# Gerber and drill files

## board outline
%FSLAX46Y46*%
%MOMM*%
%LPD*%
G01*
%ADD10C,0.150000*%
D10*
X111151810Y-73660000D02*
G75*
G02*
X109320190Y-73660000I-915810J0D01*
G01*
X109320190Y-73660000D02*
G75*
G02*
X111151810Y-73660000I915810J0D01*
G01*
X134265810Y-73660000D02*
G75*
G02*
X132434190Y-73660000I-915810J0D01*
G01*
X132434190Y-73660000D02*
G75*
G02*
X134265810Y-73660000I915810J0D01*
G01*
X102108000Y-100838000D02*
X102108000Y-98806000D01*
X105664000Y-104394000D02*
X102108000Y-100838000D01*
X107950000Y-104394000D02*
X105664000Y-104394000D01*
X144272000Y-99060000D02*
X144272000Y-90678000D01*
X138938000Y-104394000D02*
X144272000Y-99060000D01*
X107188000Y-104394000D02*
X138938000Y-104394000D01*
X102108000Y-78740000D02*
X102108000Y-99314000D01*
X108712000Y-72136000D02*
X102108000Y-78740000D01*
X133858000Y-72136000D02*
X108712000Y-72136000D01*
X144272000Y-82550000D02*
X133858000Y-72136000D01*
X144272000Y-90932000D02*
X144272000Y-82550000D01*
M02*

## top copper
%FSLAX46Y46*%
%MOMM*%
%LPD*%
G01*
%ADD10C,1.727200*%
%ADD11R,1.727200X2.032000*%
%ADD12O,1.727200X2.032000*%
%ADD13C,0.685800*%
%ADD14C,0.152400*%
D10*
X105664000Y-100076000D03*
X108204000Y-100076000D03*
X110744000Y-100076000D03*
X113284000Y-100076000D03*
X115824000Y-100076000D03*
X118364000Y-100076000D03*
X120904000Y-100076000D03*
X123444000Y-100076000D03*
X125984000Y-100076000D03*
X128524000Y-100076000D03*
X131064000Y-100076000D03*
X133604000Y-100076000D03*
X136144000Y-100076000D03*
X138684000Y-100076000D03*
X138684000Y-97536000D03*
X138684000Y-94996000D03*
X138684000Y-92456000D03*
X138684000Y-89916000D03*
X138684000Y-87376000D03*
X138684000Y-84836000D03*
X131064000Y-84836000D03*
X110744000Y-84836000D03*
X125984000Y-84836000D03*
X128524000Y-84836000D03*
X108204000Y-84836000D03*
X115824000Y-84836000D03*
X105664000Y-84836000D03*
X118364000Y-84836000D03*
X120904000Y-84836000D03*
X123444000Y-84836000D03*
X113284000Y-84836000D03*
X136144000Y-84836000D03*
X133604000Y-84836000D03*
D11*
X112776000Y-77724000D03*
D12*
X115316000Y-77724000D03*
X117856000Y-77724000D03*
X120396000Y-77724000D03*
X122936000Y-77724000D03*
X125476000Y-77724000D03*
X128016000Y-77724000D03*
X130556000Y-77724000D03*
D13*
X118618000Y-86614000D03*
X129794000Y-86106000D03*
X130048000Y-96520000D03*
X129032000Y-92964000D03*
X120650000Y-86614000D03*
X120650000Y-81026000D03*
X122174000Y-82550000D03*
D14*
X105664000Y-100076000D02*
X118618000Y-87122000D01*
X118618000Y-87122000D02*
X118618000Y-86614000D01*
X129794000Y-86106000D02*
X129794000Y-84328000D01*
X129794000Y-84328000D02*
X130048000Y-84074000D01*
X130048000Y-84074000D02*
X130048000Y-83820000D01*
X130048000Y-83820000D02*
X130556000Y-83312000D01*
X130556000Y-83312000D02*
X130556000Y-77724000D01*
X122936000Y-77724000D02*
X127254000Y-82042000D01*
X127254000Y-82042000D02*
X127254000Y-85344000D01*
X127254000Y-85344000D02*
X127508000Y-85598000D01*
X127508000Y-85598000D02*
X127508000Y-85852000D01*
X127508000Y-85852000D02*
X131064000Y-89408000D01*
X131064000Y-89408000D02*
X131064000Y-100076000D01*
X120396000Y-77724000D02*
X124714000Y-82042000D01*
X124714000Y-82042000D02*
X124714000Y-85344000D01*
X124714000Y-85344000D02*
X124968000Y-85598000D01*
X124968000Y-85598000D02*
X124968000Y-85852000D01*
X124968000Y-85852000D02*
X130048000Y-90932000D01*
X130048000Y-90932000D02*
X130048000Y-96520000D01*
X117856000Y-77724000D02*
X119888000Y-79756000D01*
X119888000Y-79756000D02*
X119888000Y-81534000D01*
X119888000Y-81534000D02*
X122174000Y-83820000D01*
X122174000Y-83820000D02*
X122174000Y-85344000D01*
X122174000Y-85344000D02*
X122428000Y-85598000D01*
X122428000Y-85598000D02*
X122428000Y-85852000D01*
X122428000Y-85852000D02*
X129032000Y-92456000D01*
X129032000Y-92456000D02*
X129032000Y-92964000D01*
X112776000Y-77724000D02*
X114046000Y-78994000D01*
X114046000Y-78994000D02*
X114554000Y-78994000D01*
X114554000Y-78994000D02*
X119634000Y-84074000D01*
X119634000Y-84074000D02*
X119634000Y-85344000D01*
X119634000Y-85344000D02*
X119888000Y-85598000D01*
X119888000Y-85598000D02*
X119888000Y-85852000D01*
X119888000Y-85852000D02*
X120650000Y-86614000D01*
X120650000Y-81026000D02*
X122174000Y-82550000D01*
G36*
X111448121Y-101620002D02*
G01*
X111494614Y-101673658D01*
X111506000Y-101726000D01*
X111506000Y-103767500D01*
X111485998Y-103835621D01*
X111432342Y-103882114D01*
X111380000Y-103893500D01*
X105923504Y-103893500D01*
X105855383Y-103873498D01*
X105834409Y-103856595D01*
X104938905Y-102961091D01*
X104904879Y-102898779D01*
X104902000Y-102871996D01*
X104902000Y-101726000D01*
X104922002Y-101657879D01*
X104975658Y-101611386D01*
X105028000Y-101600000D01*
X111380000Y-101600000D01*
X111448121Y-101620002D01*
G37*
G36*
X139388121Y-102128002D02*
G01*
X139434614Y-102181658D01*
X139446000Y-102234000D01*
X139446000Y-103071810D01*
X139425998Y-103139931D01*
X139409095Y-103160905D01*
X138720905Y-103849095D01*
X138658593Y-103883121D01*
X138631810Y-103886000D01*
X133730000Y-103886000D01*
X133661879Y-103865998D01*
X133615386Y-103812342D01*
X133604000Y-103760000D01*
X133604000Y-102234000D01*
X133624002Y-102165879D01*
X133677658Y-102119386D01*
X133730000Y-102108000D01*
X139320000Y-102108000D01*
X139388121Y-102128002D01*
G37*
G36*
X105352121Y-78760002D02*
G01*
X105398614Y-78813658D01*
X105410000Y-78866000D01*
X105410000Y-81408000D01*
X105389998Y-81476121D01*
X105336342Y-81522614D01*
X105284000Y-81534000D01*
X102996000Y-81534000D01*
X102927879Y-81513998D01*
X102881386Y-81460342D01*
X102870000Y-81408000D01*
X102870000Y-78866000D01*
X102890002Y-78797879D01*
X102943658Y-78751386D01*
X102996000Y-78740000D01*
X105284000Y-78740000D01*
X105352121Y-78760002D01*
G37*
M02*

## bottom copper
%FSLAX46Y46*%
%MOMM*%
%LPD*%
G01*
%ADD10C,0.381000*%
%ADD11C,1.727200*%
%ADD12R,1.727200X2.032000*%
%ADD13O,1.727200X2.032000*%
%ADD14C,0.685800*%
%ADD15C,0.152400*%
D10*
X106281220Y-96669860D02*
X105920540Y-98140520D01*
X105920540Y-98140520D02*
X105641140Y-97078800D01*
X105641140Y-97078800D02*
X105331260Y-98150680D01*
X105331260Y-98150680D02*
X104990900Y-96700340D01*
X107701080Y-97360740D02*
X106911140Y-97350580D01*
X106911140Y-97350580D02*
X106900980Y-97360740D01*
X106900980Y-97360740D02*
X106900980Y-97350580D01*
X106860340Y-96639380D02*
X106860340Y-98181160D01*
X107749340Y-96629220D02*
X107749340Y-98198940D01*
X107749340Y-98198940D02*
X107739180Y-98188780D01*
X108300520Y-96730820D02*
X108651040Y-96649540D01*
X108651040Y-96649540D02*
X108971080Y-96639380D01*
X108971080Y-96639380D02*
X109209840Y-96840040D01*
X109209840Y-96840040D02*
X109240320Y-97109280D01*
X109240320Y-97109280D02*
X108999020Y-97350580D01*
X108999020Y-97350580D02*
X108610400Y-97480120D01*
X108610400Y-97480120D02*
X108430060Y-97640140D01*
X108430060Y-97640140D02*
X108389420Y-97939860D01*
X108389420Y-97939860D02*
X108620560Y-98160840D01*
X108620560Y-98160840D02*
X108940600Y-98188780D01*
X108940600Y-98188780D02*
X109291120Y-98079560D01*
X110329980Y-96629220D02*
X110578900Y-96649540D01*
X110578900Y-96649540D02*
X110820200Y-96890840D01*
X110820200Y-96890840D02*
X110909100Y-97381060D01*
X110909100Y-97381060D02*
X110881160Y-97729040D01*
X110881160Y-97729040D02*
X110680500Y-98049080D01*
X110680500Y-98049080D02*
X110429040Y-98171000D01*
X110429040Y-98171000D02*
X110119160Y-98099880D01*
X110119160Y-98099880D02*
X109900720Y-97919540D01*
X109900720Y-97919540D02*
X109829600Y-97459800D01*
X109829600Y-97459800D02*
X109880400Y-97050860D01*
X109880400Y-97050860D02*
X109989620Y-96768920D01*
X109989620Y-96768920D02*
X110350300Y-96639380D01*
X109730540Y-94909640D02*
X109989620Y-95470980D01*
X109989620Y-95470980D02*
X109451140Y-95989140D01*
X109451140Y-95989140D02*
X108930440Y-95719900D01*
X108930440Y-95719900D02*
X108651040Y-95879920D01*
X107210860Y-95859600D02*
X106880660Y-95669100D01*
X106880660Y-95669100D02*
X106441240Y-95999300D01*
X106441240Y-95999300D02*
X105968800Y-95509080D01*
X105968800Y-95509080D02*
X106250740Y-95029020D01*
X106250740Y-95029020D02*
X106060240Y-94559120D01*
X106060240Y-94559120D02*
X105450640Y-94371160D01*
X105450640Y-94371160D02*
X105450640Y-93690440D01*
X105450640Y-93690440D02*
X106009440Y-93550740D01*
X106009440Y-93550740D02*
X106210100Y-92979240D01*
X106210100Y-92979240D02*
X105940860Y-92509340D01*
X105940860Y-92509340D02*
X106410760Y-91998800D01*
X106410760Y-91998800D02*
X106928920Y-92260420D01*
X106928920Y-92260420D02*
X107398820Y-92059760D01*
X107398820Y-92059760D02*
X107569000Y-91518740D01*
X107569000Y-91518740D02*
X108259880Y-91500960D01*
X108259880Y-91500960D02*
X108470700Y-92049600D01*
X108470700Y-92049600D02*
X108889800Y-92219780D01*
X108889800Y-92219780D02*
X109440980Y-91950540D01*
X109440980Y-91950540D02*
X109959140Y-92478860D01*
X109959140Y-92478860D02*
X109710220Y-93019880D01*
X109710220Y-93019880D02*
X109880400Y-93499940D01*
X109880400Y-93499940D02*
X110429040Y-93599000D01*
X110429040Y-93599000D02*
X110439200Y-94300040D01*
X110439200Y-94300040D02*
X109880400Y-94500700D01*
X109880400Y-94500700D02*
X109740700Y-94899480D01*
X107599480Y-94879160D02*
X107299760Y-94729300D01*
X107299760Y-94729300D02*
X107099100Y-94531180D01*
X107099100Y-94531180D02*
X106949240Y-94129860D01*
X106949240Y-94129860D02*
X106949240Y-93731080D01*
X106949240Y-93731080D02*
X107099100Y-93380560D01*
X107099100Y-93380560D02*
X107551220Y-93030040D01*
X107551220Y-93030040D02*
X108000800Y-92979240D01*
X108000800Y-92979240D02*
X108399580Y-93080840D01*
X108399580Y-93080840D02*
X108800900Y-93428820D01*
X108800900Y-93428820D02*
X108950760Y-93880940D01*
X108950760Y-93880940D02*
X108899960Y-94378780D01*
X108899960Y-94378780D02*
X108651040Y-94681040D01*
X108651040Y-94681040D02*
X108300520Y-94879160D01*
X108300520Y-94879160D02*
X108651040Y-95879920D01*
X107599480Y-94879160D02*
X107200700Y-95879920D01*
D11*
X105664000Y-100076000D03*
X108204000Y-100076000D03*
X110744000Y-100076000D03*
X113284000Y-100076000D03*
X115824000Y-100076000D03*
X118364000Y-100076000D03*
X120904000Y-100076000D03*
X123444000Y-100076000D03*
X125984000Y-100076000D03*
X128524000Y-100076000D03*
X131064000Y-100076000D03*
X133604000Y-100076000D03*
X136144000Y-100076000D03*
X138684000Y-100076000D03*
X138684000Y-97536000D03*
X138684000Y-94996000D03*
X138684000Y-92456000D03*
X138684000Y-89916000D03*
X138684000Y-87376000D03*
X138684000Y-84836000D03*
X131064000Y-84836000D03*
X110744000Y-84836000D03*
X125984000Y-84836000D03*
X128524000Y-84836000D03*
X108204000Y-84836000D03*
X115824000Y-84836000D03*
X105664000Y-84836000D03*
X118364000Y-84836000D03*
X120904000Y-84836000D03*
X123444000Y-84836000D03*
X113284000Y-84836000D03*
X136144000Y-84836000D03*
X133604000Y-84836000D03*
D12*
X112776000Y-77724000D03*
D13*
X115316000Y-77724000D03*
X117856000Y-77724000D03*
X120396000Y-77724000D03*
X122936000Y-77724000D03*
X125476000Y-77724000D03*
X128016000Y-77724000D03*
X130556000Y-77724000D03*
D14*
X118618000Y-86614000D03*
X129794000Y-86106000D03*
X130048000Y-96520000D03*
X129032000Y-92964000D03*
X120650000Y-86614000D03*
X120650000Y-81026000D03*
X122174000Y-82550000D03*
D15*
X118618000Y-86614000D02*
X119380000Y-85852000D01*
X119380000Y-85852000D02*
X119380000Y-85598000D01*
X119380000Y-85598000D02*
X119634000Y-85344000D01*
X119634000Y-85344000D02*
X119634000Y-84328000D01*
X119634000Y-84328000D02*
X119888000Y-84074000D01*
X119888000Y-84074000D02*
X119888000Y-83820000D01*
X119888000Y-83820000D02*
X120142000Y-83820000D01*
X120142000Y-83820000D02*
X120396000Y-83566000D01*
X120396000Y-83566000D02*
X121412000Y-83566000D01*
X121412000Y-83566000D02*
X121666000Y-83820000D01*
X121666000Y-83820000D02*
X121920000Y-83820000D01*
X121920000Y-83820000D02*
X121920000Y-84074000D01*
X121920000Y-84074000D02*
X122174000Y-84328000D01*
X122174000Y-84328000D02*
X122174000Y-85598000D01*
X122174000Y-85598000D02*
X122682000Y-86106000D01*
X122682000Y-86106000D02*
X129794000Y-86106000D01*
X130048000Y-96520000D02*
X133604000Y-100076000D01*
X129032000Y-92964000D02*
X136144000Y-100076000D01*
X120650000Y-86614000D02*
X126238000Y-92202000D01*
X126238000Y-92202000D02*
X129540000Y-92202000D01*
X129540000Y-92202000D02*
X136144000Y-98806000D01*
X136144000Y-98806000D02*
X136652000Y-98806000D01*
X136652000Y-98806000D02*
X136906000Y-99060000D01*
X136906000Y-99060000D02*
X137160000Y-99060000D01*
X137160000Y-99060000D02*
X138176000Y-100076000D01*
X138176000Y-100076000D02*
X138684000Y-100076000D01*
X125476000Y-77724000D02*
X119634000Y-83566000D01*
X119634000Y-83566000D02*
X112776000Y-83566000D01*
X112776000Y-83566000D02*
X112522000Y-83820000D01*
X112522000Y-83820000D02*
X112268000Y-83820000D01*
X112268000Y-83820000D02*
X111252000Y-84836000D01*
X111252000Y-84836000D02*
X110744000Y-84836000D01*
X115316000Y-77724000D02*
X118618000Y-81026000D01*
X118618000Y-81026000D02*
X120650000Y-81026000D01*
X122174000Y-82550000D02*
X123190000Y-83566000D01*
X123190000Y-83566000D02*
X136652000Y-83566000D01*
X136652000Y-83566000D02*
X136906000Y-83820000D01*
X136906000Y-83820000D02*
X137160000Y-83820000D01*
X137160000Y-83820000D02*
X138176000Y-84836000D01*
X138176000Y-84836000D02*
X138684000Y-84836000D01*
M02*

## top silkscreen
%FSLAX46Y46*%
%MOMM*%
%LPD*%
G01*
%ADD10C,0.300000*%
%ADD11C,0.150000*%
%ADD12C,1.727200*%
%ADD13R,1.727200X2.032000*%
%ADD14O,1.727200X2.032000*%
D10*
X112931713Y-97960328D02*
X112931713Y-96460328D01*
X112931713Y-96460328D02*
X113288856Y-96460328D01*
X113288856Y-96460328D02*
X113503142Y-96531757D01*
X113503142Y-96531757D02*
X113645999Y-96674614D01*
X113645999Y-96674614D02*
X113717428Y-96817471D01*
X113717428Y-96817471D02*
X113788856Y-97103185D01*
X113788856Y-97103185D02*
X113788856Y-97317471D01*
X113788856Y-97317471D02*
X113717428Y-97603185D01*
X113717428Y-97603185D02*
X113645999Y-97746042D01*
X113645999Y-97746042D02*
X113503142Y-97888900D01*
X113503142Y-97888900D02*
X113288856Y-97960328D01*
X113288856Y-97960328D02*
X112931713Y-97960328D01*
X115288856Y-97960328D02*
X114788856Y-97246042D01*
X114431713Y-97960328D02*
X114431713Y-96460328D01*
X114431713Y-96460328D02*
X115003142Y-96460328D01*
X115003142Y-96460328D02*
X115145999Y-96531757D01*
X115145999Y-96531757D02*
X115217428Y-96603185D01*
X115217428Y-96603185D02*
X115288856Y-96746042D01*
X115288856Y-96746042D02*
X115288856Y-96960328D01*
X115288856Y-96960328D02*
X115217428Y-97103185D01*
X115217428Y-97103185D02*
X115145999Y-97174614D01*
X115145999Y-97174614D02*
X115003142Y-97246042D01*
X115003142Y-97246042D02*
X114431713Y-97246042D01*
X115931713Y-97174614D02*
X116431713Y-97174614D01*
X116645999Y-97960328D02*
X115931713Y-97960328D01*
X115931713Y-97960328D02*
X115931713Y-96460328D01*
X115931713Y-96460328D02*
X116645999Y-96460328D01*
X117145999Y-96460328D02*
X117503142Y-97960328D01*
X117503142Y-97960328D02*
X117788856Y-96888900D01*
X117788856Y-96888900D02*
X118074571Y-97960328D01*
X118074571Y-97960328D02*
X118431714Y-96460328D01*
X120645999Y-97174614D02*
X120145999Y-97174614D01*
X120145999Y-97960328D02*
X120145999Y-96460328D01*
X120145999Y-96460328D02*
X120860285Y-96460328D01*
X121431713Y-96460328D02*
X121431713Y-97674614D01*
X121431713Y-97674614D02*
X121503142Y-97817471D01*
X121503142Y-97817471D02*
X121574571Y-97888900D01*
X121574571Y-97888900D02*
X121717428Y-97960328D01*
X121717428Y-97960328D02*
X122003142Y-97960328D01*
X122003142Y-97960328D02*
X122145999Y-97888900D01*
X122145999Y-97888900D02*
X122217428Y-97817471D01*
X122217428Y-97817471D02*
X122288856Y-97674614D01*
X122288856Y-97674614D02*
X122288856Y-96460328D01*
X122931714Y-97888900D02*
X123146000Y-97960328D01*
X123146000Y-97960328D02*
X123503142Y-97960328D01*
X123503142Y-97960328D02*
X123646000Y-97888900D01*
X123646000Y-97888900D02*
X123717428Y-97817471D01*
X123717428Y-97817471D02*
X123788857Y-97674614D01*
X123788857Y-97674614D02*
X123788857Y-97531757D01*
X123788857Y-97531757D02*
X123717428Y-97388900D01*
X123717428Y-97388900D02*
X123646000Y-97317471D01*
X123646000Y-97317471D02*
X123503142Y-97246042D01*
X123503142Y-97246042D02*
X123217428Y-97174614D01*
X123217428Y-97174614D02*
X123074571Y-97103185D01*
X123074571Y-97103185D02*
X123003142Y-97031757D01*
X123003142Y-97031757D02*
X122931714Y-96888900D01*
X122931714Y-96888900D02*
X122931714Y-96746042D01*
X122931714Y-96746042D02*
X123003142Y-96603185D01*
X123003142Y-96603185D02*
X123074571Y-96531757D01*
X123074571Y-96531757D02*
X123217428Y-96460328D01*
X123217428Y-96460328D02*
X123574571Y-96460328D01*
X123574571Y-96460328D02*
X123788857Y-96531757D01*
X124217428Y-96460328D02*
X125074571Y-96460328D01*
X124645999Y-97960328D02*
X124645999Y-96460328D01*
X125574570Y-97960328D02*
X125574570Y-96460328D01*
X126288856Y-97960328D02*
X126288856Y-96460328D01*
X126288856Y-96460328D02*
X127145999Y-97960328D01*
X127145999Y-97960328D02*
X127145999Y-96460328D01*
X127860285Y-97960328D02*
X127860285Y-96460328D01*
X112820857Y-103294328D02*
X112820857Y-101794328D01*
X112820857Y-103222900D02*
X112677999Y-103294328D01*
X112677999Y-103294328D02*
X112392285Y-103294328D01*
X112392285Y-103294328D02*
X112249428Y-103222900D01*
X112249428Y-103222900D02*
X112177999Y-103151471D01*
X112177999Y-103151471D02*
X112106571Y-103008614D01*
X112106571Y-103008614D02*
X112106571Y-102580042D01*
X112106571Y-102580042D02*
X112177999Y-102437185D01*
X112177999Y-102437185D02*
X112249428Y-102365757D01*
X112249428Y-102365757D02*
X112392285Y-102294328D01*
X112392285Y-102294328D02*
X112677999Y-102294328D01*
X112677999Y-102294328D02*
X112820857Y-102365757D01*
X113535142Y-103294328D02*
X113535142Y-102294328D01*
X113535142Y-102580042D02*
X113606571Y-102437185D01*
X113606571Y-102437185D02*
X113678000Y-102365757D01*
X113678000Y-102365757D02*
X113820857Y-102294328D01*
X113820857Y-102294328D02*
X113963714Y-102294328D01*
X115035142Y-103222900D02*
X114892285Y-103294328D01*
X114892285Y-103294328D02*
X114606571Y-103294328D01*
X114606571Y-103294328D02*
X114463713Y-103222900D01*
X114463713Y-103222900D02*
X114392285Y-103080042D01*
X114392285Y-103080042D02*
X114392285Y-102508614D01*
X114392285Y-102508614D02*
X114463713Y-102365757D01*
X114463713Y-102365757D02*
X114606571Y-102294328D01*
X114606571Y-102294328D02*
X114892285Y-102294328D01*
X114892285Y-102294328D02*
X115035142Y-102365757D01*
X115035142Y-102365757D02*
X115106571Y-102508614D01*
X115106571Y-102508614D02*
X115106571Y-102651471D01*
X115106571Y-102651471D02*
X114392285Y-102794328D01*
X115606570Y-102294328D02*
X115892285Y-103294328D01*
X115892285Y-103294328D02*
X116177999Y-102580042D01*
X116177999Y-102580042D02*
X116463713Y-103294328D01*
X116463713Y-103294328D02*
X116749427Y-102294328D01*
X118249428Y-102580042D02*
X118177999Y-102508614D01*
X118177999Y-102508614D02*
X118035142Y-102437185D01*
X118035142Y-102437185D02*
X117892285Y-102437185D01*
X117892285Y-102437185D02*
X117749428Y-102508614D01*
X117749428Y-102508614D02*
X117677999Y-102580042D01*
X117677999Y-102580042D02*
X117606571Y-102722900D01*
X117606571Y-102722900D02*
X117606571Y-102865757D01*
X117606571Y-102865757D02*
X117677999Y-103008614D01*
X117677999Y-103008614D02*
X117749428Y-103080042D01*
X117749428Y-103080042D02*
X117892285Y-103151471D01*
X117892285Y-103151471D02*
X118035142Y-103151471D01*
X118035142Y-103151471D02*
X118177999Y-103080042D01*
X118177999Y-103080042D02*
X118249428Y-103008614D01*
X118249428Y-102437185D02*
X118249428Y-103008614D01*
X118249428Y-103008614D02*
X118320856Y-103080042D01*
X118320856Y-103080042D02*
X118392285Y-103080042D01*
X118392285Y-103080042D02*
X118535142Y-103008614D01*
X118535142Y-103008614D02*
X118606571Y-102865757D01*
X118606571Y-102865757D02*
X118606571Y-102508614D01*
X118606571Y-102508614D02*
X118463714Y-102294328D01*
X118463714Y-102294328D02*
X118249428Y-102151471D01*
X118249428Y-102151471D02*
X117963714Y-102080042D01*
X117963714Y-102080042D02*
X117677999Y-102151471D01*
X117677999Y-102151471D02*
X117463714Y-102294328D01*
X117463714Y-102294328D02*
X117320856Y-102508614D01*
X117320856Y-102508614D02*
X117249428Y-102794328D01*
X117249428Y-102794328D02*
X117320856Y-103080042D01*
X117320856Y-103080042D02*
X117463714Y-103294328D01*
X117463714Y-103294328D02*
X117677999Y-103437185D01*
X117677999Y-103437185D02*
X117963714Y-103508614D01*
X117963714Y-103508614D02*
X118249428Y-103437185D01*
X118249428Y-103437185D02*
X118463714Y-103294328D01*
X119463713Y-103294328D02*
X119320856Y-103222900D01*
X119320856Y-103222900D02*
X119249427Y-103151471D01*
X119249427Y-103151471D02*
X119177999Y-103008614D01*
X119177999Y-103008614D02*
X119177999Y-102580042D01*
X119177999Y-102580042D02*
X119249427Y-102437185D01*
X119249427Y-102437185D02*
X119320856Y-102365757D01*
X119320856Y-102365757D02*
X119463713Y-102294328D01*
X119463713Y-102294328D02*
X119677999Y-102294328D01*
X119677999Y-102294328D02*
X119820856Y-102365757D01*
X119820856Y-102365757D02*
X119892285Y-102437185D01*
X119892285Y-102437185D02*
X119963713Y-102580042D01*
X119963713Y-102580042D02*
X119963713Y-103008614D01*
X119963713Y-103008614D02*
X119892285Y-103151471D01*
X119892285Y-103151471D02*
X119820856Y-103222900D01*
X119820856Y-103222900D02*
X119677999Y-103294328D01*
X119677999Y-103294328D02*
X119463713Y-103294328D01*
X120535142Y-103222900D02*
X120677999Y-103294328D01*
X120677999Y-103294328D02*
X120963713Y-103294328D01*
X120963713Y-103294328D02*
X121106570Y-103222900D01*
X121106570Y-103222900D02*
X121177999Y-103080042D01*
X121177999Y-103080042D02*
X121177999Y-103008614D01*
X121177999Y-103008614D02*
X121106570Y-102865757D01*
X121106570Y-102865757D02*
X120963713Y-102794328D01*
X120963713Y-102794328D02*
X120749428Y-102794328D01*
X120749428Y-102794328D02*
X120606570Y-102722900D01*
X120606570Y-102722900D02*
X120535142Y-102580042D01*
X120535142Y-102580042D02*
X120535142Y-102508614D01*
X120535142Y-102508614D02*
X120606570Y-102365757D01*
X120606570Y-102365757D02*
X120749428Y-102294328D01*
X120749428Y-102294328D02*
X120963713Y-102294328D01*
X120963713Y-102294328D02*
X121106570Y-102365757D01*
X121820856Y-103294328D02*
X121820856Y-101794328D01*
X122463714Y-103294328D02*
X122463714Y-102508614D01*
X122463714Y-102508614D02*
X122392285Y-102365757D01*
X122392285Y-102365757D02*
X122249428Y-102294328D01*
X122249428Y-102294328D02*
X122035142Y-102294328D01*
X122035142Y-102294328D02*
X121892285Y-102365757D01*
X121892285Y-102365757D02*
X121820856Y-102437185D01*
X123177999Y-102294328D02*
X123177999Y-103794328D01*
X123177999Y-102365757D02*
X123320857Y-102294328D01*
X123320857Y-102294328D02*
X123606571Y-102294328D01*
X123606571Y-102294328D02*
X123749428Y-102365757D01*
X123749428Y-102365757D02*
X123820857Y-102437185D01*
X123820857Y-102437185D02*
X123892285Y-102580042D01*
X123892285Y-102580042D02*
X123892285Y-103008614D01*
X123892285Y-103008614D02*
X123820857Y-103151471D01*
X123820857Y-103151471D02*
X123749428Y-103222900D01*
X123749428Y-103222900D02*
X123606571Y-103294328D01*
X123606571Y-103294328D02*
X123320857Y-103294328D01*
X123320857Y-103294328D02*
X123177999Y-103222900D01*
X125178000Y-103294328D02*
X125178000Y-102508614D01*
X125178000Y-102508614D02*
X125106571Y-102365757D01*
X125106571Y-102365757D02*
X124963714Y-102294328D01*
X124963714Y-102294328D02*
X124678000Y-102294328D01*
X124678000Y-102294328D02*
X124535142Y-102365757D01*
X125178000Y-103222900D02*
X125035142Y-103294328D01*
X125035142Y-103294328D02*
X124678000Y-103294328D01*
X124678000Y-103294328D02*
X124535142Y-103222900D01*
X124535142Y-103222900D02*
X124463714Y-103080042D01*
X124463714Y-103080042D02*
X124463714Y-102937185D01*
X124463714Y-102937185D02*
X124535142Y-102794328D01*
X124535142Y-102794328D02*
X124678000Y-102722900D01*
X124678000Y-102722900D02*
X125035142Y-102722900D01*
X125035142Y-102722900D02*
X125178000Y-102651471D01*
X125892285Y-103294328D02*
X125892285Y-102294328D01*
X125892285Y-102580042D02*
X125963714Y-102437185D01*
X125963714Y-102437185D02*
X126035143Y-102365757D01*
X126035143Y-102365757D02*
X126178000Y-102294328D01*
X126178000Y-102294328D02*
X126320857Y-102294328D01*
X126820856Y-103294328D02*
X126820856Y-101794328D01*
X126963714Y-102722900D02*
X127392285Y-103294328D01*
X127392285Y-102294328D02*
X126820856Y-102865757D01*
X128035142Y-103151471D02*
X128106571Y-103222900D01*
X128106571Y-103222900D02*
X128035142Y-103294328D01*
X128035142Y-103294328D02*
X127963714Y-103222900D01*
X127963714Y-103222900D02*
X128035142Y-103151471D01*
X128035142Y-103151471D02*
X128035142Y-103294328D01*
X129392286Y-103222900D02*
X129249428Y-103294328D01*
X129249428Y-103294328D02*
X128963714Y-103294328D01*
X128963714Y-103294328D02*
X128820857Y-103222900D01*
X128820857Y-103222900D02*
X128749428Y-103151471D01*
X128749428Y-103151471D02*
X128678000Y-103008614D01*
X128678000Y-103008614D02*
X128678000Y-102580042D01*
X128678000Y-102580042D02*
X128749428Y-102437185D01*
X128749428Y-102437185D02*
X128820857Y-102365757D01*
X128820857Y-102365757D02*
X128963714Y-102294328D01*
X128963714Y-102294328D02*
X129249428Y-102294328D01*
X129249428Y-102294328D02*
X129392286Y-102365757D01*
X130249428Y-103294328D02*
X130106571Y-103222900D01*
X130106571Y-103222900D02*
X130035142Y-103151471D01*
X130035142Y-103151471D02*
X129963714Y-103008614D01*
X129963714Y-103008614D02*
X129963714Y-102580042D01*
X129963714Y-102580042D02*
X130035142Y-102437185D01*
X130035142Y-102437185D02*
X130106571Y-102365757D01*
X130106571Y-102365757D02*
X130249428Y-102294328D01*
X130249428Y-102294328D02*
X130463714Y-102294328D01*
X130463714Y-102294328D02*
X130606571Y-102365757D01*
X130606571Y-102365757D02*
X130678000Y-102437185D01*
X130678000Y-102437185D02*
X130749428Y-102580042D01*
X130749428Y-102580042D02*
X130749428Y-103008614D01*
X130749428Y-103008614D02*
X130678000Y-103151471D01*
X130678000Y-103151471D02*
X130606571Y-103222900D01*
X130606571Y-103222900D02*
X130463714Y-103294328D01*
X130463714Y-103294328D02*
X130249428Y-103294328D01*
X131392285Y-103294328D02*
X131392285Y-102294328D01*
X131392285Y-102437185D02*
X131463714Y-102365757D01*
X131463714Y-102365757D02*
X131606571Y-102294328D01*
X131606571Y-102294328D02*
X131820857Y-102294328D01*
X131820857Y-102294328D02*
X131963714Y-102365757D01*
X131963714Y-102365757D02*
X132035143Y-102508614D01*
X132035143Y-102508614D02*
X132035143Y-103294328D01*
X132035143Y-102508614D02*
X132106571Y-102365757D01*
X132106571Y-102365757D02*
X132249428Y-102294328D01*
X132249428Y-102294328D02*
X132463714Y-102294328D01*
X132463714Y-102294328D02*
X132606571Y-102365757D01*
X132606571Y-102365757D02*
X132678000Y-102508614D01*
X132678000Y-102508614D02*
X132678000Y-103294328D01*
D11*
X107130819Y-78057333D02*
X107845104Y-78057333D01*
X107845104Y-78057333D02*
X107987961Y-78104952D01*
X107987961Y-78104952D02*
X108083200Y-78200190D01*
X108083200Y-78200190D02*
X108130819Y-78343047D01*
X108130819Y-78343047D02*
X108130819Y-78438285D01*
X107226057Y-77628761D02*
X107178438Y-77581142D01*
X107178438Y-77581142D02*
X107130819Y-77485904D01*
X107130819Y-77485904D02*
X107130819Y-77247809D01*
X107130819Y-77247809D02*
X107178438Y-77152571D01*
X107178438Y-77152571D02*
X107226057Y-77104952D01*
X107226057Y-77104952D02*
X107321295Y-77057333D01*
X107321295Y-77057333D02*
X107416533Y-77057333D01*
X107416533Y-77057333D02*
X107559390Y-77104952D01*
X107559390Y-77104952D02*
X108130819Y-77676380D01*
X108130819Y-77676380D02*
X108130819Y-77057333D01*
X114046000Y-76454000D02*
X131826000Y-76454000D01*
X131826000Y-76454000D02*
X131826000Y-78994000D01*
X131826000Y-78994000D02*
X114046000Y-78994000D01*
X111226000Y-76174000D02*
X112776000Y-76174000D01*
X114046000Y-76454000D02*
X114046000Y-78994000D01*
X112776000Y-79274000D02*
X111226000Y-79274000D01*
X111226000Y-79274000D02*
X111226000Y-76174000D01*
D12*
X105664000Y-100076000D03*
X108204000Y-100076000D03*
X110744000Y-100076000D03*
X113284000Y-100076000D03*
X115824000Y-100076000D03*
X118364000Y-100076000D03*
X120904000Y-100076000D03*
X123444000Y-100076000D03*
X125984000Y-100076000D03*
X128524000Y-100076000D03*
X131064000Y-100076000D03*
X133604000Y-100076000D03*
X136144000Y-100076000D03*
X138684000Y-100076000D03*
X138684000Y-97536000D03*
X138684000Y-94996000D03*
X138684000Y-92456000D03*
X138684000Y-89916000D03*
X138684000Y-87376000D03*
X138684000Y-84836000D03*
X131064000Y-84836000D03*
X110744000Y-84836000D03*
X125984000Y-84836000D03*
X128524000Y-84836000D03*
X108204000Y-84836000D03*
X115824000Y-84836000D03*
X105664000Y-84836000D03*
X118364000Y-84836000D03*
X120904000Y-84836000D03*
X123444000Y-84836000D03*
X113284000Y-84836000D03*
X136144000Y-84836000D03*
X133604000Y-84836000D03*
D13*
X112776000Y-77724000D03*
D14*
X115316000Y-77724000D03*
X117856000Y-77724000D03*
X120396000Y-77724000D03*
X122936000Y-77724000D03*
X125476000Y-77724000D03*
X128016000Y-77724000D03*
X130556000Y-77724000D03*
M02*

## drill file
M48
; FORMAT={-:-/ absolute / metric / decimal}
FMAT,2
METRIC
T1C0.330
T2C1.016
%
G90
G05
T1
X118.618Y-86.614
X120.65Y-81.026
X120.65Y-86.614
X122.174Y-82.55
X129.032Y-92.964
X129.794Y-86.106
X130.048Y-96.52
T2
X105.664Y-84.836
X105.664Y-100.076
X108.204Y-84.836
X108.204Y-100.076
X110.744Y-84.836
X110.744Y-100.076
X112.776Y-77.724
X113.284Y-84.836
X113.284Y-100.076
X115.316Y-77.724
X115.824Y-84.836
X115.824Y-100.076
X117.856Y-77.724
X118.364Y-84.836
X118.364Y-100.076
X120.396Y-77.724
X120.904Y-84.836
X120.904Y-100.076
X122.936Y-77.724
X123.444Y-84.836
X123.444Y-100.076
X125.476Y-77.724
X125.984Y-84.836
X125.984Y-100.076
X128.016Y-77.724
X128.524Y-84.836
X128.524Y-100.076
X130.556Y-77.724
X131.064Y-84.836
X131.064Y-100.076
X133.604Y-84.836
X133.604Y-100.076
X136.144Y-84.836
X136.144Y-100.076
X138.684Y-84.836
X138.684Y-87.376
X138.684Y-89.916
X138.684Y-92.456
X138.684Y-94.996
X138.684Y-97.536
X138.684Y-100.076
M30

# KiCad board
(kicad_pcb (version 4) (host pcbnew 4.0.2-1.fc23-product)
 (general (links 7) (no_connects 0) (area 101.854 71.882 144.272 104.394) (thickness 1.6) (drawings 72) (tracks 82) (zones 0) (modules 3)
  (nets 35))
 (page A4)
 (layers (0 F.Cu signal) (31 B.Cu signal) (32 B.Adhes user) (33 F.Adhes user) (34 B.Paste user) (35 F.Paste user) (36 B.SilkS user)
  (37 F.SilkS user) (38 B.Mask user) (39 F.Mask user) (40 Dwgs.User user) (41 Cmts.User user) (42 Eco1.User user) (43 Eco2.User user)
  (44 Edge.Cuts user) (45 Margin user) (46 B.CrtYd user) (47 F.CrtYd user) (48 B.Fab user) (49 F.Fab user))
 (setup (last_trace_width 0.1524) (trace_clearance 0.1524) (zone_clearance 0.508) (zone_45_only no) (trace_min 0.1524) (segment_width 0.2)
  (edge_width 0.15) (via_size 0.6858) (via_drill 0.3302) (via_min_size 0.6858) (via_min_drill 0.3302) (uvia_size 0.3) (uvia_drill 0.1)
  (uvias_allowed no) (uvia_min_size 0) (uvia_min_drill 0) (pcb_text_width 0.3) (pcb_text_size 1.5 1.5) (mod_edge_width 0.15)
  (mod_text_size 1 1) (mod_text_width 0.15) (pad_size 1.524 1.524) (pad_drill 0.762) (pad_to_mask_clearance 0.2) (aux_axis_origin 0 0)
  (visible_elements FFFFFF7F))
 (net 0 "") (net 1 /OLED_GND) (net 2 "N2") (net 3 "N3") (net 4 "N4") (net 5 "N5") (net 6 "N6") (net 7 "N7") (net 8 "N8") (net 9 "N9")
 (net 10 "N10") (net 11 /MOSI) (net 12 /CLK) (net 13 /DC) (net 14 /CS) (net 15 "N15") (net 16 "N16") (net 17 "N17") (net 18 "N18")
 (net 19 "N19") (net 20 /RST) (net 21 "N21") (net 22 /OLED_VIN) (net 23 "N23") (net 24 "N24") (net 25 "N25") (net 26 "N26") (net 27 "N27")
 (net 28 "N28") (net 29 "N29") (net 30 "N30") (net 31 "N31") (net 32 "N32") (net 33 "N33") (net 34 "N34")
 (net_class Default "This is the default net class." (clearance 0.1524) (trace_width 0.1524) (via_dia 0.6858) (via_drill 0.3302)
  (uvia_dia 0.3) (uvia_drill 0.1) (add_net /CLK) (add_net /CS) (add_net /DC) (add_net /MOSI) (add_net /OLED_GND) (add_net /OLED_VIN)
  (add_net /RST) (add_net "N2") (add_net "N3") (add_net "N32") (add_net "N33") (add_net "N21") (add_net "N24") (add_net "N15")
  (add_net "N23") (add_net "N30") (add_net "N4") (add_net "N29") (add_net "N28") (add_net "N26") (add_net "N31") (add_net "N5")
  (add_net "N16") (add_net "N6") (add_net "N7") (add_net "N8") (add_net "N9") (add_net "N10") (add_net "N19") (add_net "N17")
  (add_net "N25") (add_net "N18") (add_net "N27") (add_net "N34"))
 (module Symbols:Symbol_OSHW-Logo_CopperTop (layer B.Cu) (at 107.95 93.98 180)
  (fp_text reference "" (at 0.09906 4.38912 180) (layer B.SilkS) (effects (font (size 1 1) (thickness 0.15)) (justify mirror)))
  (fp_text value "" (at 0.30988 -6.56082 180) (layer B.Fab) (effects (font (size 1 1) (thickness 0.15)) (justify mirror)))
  (fp_line (start 1.66878 -2.68986) (end 2.02946 -4.16052) (layer B.Cu) (width 0.381))
  (fp_line (start 2.02946 -4.16052) (end 2.30886 -3.0988) (layer B.Cu) (width 0.381))
  (fp_line (start 2.30886 -3.0988) (end 2.61874 -4.17068) (layer B.Cu) (width 0.381))
  (fp_line (start 2.61874 -4.17068) (end 2.9591 -2.72034) (layer B.Cu) (width 0.381))
  (fp_line (start 0.24892 -3.38074) (end 1.03886 -3.37058) (layer B.Cu) (width 0.381))
  (fp_line (start 1.03886 -3.37058) (end 1.04902 -3.38074) (layer B.Cu) (width 0.381))
  (fp_line (start 1.04902 -3.38074) (end 1.04902 -3.37058) (layer B.Cu) (width 0.381))
  (fp_line (start 1.08966 -2.65938) (end 1.08966 -4.20116) (layer B.Cu) (width 0.381))
  (fp_line (start 0.20066 -2.64922) (end 0.20066 -4.21894) (layer B.Cu) (width 0.381))
  (fp_line (start 0.20066 -4.21894) (end 0.21082 -4.20878) (layer B.Cu) (width 0.381))
  (fp_line (start -0.35052 -2.75082) (end -0.70104 -2.66954) (layer B.Cu) (width 0.381))
  (fp_line (start -0.70104 -2.66954) (end -1.02108 -2.65938) (layer B.Cu) (width 0.381))
  (fp_line (start -1.02108 -2.65938) (end -1.25984 -2.86004) (layer B.Cu) (width 0.381))
  (fp_line (start -1.25984 -2.86004) (end -1.29032 -3.12928) (layer B.Cu) (width 0.381))
  (fp_line (start -1.29032 -3.12928) (end -1.04902 -3.37058) (layer B.Cu) (width 0.381))
  (fp_line (start -1.04902 -3.37058) (end -0.6604 -3.50012) (layer B.Cu) (width 0.381))
  (fp_line (start -0.6604 -3.50012) (end -0.48006 -3.66014) (layer B.Cu) (width 0.381))
  (fp_line (start -0.48006 -3.66014) (end -0.43942 -3.95986) (layer B.Cu) (width 0.381))
  (fp_line (start -0.43942 -3.95986) (end -0.67056 -4.18084) (layer B.Cu) (width 0.381))
  (fp_line (start -0.67056 -4.18084) (end -0.9906 -4.20878) (layer B.Cu) (width 0.381))
  (fp_line (start -0.9906 -4.20878) (end -1.34112 -4.09956) (layer B.Cu) (width 0.381))
  (fp_line (start -2.37998 -2.64922) (end -2.6289 -2.66954) (layer B.Cu) (width 0.381))
  (fp_line (start -2.6289 -2.66954) (end -2.8702 -2.91084) (layer B.Cu) (width 0.381))
  (fp_line (start -2.8702 -2.91084) (end -2.9591 -3.40106) (layer B.Cu) (width 0.381))
  (fp_line (start -2.9591 -3.40106) (end -2.93116 -3.74904) (layer B.Cu) (width 0.381))
  (fp_line (start -2.93116 -3.74904) (end -2.7305 -4.06908) (layer B.Cu) (width 0.381))
  (fp_line (start -2.7305 -4.06908) (end -2.47904 -4.191) (layer B.Cu) (width 0.381))
  (fp_line (start -2.47904 -4.191) (end -2.16916 -4.11988) (layer B.Cu) (width 0.381))
  (fp_line (start -2.16916 -4.11988) (end -1.95072 -3.93954) (layer B.Cu) (width 0.381))
  (fp_line (start -1.95072 -3.93954) (end -1.8796 -3.4798) (layer B.Cu) (width 0.381))
  (fp_line (start -1.8796 -3.4798) (end -1.9304 -3.07086) (layer B.Cu) (width 0.381))
  (fp_line (start -1.9304 -3.07086) (end -2.03962 -2.78892) (layer B.Cu) (width 0.381))
  (fp_line (start -2.03962 -2.78892) (end -2.4003 -2.65938) (layer B.Cu) (width 0.381))
  (fp_line (start -1.78054 -0.92964) (end -2.03962 -1.49098) (layer B.Cu) (width 0.381))
  (fp_line (start -2.03962 -1.49098) (end -1.50114 -2.00914) (layer B.Cu) (width 0.381))
  (fp_line (start -1.50114 -2.00914) (end -0.98044 -1.7399) (layer B.Cu) (width 0.381))
  (fp_line (start -0.98044 -1.7399) (end -0.70104 -1.89992) (layer B.Cu) (width 0.381))
  (fp_line (start 0.73914 -1.8796) (end 1.06934 -1.6891) (layer B.Cu) (width 0.381))
  (fp_line (start 1.06934 -1.6891) (end 1.50876 -2.0193) (layer B.Cu) (width 0.381))
  (fp_line (start 1.50876 -2.0193) (end 1.9812 -1.52908) (layer B.Cu) (width 0.381))
  (fp_line (start 1.9812 -1.52908) (end 1.69926 -1.04902) (layer B.Cu) (width 0.381))
  (fp_line (start 1.69926 -1.04902) (end 1.88976 -0.57912) (layer B.Cu) (width 0.381))
  (fp_line (start 1.88976 -0.57912) (end 2.49936 -0.39116) (layer B.Cu) (width 0.381))
  (fp_line (start 2.49936 -0.39116) (end 2.49936 0.28956) (layer B.Cu) (width 0.381))
  (fp_line (start 2.49936 0.28956) (end 1.94056 0.42926) (layer B.Cu) (width 0.381))
  (fp_line (start 1.94056 0.42926) (end 1.7399 1.00076) (layer B.Cu) (width 0.381))
  (fp_line (start 1.7399 1.00076) (end 2.00914 1.47066) (layer B.Cu) (width 0.381))
  (fp_line (start 2.00914 1.47066) (end 1.53924 1.9812) (layer B.Cu) (width 0.381))
  (fp_line (start 1.53924 1.9812) (end 1.02108 1.71958) (layer B.Cu) (width 0.381))
  (fp_line (start 1.02108 1.71958) (end 0.55118 1.92024) (layer B.Cu) (width 0.381))
  (fp_line (start 0.55118 1.92024) (end 0.381 2.46126) (layer B.Cu) (width 0.381))
  (fp_line (start 0.381 2.46126) (end -0.30988 2.47904) (layer B.Cu) (width 0.381))
  (fp_line (start -0.30988 2.47904) (end -0.5207 1.9304) (layer B.Cu) (width 0.381))
  (fp_line (start -0.5207 1.9304) (end -0.9398 1.76022) (layer B.Cu) (width 0.381))
  (fp_line (start -0.9398 1.76022) (end -1.49098 2.02946) (layer B.Cu) (width 0.381))
  (fp_line (start -1.49098 2.02946) (end -2.00914 1.50114) (layer B.Cu) (width 0.381))
  (fp_line (start -2.00914 1.50114) (end -1.76022 0.96012) (layer B.Cu) (width 0.381))
  (fp_line (start -1.76022 0.96012) (end -1.9304 0.48006) (layer B.Cu) (width 0.381))
  (fp_line (start -1.9304 0.48006) (end -2.47904 0.381) (layer B.Cu) (width 0.381))
  (fp_line (start -2.47904 0.381) (end -2.4892 -0.32004) (layer B.Cu) (width 0.381))
  (fp_line (start -2.4892 -0.32004) (end -1.9304 -0.5207) (layer B.Cu) (width 0.381))
  (fp_line (start -1.9304 -0.5207) (end -1.7907 -0.91948) (layer B.Cu) (width 0.381))
  (fp_line (start 0.35052 -0.89916) (end 0.65024 -0.7493) (layer B.Cu) (width 0.381))
  (fp_line (start 0.65024 -0.7493) (end 0.8509 -0.55118) (layer B.Cu) (width 0.381))
  (fp_line (start 0.8509 -0.55118) (end 1.00076 -0.14986) (layer B.Cu) (width 0.381))
  (fp_line (start 1.00076 -0.14986) (end 1.00076 0.24892) (layer B.Cu) (width 0.381))
  (fp_line (start 1.00076 0.24892) (end 0.8509 0.59944) (layer B.Cu) (width 0.381))
  (fp_line (start 0.8509 0.59944) (end 0.39878 0.94996) (layer B.Cu) (width 0.381))
  (fp_line (start 0.39878 0.94996) (end -0.0508 1.00076) (layer B.Cu) (width 0.381))
  (fp_line (start -0.0508 1.00076) (end -0.44958 0.89916) (layer B.Cu) (width 0.381))
  (fp_line (start -0.44958 0.89916) (end -0.8509 0.55118) (layer B.Cu) (width 0.381))
  (fp_line (start -0.8509 0.55118) (end -1.00076 0.09906) (layer B.Cu) (width 0.381))
  (fp_line (start -1.00076 0.09906) (end -0.94996 -0.39878) (layer B.Cu) (width 0.381))
  (fp_line (start -0.94996 -0.39878) (end -0.70104 -0.70104) (layer B.Cu) (width 0.381))
  (fp_line (start -0.70104 -0.70104) (end -0.35052 -0.89916) (layer B.Cu) (width 0.381))
  (fp_line (start -0.35052 -0.89916) (end -0.70104 -1.89992) (layer B.Cu) (width 0.381))
  (fp_line (start 0.35052 -0.89916) (end 0.7493 -1.89992) (layer B.Cu) (width 0.381)))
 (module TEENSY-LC (layer F.Cu) (at 115.824 89.916 90)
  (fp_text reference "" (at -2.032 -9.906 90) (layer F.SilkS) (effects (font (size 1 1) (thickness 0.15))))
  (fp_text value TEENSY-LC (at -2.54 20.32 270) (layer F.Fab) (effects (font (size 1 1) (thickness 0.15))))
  (pad G1 thru_hole circle (at -10.16 -10.16 90) (size 1.7272 1.7272) (drill 1.016) (layers *.Cu *.Mask F.SilkS) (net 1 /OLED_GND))
  (pad 0 thru_hole circle (at -10.16 -7.62 90) (size 1.7272 1.7272) (drill 1.016) (layers *.Cu *.Mask F.SilkS) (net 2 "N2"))
  (pad 1 thru_hole circle (at -10.16 -5.08 90) (size 1.7272 1.7272) (drill 1.016) (layers *.Cu *.Mask F.SilkS) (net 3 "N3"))
  (pad 2 thru_hole circle (at -10.16 -2.54 90) (size 1.7272 1.7272) (drill 1.016) (layers *.Cu *.Mask F.SilkS) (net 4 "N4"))
  (pad 3 thru_hole circle (at -10.16 0 90) (size 1.7272 1.7272) (drill 1.016) (layers *.Cu *.Mask F.SilkS) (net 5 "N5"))
  (pad 4 thru_hole circle (at -10.16 2.54 90) (size 1.7272 1.7272) (drill 1.016) (layers *.Cu *.Mask F.SilkS) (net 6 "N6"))
  (pad 5 thru_hole circle (at -10.16 5.08 90) (size 1.7272 1.7272) (drill 1.016) (layers *.Cu *.Mask F.SilkS) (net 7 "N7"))
  (pad 6 thru_hole circle (at -10.16 7.62 90) (size 1.7272 1.7272) (drill 1.016) (layers *.Cu *.Mask F.SilkS) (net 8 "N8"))
  (pad 7 thru_hole circle (at -10.16 10.16 90) (size 1.7272 1.7272) (drill 1.016) (layers *.Cu *.Mask F.SilkS) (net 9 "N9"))
  (pad 8 thru_hole circle (at -10.16 12.7 90) (size 1.7272 1.7272) (drill 1.016) (layers *.Cu *.Mask F.SilkS) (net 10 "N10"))
  (pad 9 thru_hole circle (at -10.16 15.24 90) (size 1.7272 1.7272) (drill 1.016) (layers *.Cu *.Mask F.SilkS) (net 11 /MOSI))
  (pad 10 thru_hole circle (at -10.16 17.78 90) (size 1.7272 1.7272) (drill 1.016) (layers *.Cu *.Mask F.SilkS) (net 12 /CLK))
  (pad 11 thru_hole circle (at -10.16 20.32 90) (size 1.7272 1.7272) (drill 1.016) (layers *.Cu *.Mask F.SilkS) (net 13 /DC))
  (pad 12 thru_hole circle (at -10.16 22.86 90) (size 1.7272 1.7272) (drill 1.016) (layers *.Cu *.Mask F.SilkS) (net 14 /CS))
  (pad 17A thru_hole circle (at -7.62 22.86 90) (size 1.7272 1.7272) (drill 1.016) (layers *.Cu *.Mask F.SilkS) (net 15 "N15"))
  (pad 3V1 thru_hole circle (at -5.08 22.86 90) (size 1.7272 1.7272) (drill 1.016) (layers *.Cu *.Mask F.SilkS) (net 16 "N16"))
  (pad G2 thru_hole circle (at -2.54 22.86 90) (size 1.7272 1.7272) (drill 1.016) (layers *.Cu *.Mask F.SilkS) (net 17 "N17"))
  (pad PGM thru_hole circle (at 0 22.86 90) (size 1.7272 1.7272) (drill 1.016) (layers *.Cu *.Mask F.SilkS) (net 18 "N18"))
  (pad DAC thru_hole circle (at 2.54 22.86 90) (size 1.7272 1.7272) (drill 1.016) (layers *.Cu *.Mask F.SilkS) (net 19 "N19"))
  (pad 13 thru_hole circle (at 5.08 22.86 90) (size 1.7272 1.7272) (drill 1.016) (layers *.Cu *.Mask F.SilkS) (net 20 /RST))
  (pad 16 thru_hole circle (at 5.08 15.24 90) (size 1.7272 1.7272) (drill 1.016) (layers *.Cu *.Mask F.SilkS) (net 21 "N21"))
  (pad 3V2 thru_hole circle (at 5.08 -5.08 90) (size 1.7272 1.7272) (drill 1.016) (layers *.Cu *.Mask F.SilkS) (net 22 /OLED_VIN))
  (pad 18 thru_hole circle (at 5.08 10.16 90) (size 1.7272 1.7272) (drill 1.016) (layers *.Cu *.Mask F.SilkS) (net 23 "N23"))
  (pad 17 thru_hole circle (at 5.08 12.7 90) (size 1.7272 1.7272) (drill 1.016) (layers *.Cu *.Mask F.SilkS) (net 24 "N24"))
  (pad G3 thru_hole circle (at 5.08 -7.62 90) (size 1.7272 1.7272) (drill 1.016) (layers *.Cu *.Mask F.SilkS) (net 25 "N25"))
  (pad 22 thru_hole circle (at 5.08 0 90) (size 1.7272 1.7272) (drill 1.016) (layers *.Cu *.Mask F.SilkS) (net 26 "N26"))
  (pad VIN thru_hole circle (at 5.08 -10.16 90) (size 1.7272 1.7272) (drill 1.016) (layers *.Cu *.Mask F.SilkS) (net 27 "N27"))
  (pad 21 thru_hole circle (at 5.08 2.54 90) (size 1.7272 1.7272) (drill 1.016) (layers *.Cu *.Mask F.SilkS) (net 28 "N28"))
  (pad 20 thru_hole circle (at 5.08 5.08 90) (size 1.7272 1.7272) (drill 1.016) (layers *.Cu *.Mask F.SilkS) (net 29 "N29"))
  (pad 19 thru_hole circle (at 5.08 7.62 90) (size 1.7272 1.7272) (drill 1.016) (layers *.Cu *.Mask F.SilkS) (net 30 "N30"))
  (pad 23 thru_hole circle (at 5.08 -2.54 90) (size 1.7272 1.7272) (drill 1.016) (layers *.Cu *.Mask F.SilkS) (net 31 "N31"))
  (pad 14 thru_hole circle (at 5.08 20.32 90) (size 1.7272 1.7272) (drill 1.016) (layers *.Cu *.Mask F.SilkS) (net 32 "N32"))
  (pad 15 thru_hole circle (at 5.08 17.78 90) (size 1.7272 1.7272) (drill 1.016) (layers *.Cu *.Mask F.SilkS) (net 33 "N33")))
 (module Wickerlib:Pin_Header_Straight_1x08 (layer F.Cu) (at 112.776 77.724 90)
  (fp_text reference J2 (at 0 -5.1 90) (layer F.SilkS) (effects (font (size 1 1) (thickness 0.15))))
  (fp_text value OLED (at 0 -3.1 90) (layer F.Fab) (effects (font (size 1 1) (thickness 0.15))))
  (fp_line (start 1.27 1.27) (end 1.27 19.05) (layer F.SilkS) (width 0.15))
  (fp_line (start 1.27 19.05) (end -1.27 19.05) (layer F.SilkS) (width 0.15))
  (fp_line (start -1.27 19.05) (end -1.27 1.27) (layer F.SilkS) (width 0.15))
  (fp_line (start 1.55 -1.55) (end 1.55 0) (layer F.SilkS) (width 0.15))
  (fp_line (start 1.27 1.27) (end -1.27 1.27) (layer F.SilkS) (width 0.15))
  (fp_line (start -1.55 0) (end -1.55 -1.55) (layer F.SilkS) (width 0.15))
  (fp_line (start -1.55 -1.55) (end 1.55 -1.55) (layer F.SilkS) (width 0.15))
  (pad 1 thru_hole rect (at 0 0 90) (size 2.032 1.7272) (drill 1.016) (layers *.Cu *.Mask F.SilkS) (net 14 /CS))
  (pad 2 thru_hole oval (at 0 2.54 90) (size 2.032 1.7272) (drill 1.016) (layers *.Cu *.Mask F.SilkS) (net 20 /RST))
  (pad 3 thru_hole oval (at 0 5.08 90) (size 2.032 1.7272) (drill 1.016) (layers *.Cu *.Mask F.SilkS) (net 13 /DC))
  (pad 4 thru_hole oval (at 0 7.62 90) (size 2.032 1.7272) (drill 1.016) (layers *.Cu *.Mask F.SilkS) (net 12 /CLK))
  (pad 5 thru_hole oval (at 0 10.16 90) (size 2.032 1.7272) (drill 1.016) (layers *.Cu *.Mask F.SilkS) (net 11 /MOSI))
  (pad 6 thru_hole oval (at 0 12.7 90) (size 2.032 1.7272) (drill 1.016) (layers *.Cu *.Mask F.SilkS) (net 22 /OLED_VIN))
  (pad 7 thru_hole oval (at 0 15.24 90) (size 2.032 1.7272) (drill 1.016) (layers *.Cu *.Mask F.SilkS) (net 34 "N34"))
  (pad 8 thru_hole oval (at 0 17.78 90) (size 2.032 1.7272) (drill 1.016) (layers *.Cu *.Mask F.SilkS) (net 1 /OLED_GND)))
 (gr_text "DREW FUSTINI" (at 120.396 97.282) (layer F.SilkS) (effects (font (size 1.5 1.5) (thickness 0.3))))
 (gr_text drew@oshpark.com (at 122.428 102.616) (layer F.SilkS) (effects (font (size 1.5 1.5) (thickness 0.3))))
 (gr_circle (center 110.236 73.66) (end 110.744 74.422) (layer Edge.Cuts) (width 0.15))
 (gr_circle (center 133.35 73.66) (end 132.588 73.152) (layer Edge.Cuts) (width 0.15))
 (gr_line (start 102.108 100.838) (end 102.108 98.806) (angle 90) (layer Edge.Cuts) (width 0.15))
 (gr_line (start 105.664 104.394) (end 102.108 100.838) (angle 90) (layer Edge.Cuts) (width 0.15))
 (gr_line (start 107.95 104.394) (end 105.664 104.394) (angle 90) (layer Edge.Cuts) (width 0.15))
 (gr_line (start 144.272 99.06) (end 144.272 90.678) (angle 90) (layer Edge.Cuts) (width 0.15))
 (gr_line (start 138.938 104.394) (end 144.272 99.06) (angle 90) (layer Edge.Cuts) (width 0.15))
 (gr_line (start 107.188 104.394) (end 138.938 104.394) (angle 90) (layer Edge.Cuts) (width 0.15))
 (gr_line (start 102.108 78.74) (end 102.108 99.314) (angle 90) (layer Edge.Cuts) (width 0.15))
 (gr_line (start 108.712 72.136) (end 102.108 78.74) (angle 90) (layer Edge.Cuts) (width 0.15))
 (gr_line (start 133.858 72.136) (end 108.712 72.136) (angle 90) (layer Edge.Cuts) (width 0.15))
 (gr_line (start 144.272 82.55) (end 133.858 72.136) (angle 90) (layer Edge.Cuts) (width 0.15))
 (gr_line (start 144.272 90.932) (end 144.272 82.55) (angle 90) (layer Edge.Cuts) (width 0.15))
 (segment (start 105.664 100.076) (end 118.618 87.122) (width 0.1524) (layer F.Cu) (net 1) (status 80000))
 (segment (start 118.618 87.122) (end 118.618 86.614) (width 0.1524) (layer F.Cu) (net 1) (status 80000))
 (via (at 118.618 86.614) (size 0.6858) (layers F.Cu B.Cu) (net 1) (status 80000))
 (segment (start 118.618 86.614) (end 119.38 85.852) (width 0.1524) (layer B.Cu) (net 1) (status 80000))
 (segment (start 119.38 85.852) (end 119.38 85.598) (width 0.1524) (layer B.Cu) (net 1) (status 80000))
 (segment (start 119.38 85.598) (end 119.634 85.344) (width 0.1524) (layer B.Cu) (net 1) (status 80000))
 (segment (start 119.634 85.344) (end 119.634 84.328) (width 0.1524) (layer B.Cu) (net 1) (status 80000))
 (segment (start 119.634 84.328) (end 119.888 84.074) (width 0.1524) (layer B.Cu) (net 1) (status 80000))
 (segment (start 119.888 84.074) (end 119.888 83.82) (width 0.1524) (layer B.Cu) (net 1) (status 80000))
 (segment (start 119.888 83.82) (end 120.142 83.82) (width 0.1524) (layer B.Cu) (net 1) (status 80000))
 (segment (start 120.142 83.82) (end 120.396 83.566) (width 0.1524) (layer B.Cu) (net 1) (status 80000))
 (segment (start 120.396 83.566) (end 121.412 83.566) (width 0.1524) (layer B.Cu) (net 1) (status 80000))
 (segment (start 121.412 83.566) (end 121.666 83.82) (width 0.1524) (layer B.Cu) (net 1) (status 80000))
 (segment (start 121.666 83.82) (end 121.92 83.82) (width 0.1524) (layer B.Cu) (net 1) (status 80000))
 (segment (start 121.92 83.82) (end 121.92 84.074) (width 0.1524) (layer B.Cu) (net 1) (status 80000))
 (segment (start 121.92 84.074) (end 122.174 84.328) (width 0.1524) (layer B.Cu) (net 1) (status 80000))
 (segment (start 122.174 84.328) (end 122.174 85.598) (width 0.1524) (layer B.Cu) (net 1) (status 80000))
 (segment (start 122.174 85.598) (end 122.682 86.106) (width 0.1524) (layer B.Cu) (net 1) (status 80000))
 (segment (start 122.682 86.106) (end 129.794 86.106) (width 0.1524) (layer B.Cu) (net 1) (status 80000))
 (via (at 129.794 86.106) (size 0.6858) (layers F.Cu B.Cu) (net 1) (status 80000))
 (segment (start 129.794 86.106) (end 129.794 84.328) (width 0.1524) (layer F.Cu) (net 1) (status 80000))
 (segment (start 129.794 84.328) (end 130.048 84.074) (width 0.1524) (layer F.Cu) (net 1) (status 80000))
 (segment (start 130.048 84.074) (end 130.048 83.82) (width 0.1524) (layer F.Cu) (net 1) (status 80000))
 (segment (start 130.048 83.82) (end 130.556 83.312) (width 0.1524) (layer F.Cu) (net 1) (status 80000))
 (segment (start 130.556 83.312) (end 130.556 77.724) (width 0.1524) (layer F.Cu) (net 1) (status 80000))
 (segment (start 122.936 77.724) (end 127.254 82.042) (width 0.1524) (layer F.Cu) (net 11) (status 80000))
 (segment (start 127.254 82.042) (end 127.254 85.344) (width 0.1524) (layer F.Cu) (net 11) (status 80000))
 (segment (start 127.254 85.344) (end 127.508 85.598) (width 0.1524) (layer F.Cu) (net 11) (status 80000))
 (segment (start 127.508 85.598) (end 127.508 85.852) (width 0.1524) (layer F.Cu) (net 11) (status 80000))
 (segment (start 127.508 85.852) (end 131.064 89.408) (width 0.1524) (layer F.Cu) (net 11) (status 80000))
 (segment (start 131.064 89.408) (end 131.064 100.076) (width 0.1524) (layer F.Cu) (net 11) (status 80000))
 (segment (start 120.396 77.724) (end 124.714 82.042) (width 0.1524) (layer F.Cu) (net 12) (status 80000))
 (segment (start 124.714 82.042) (end 124.714 85.344) (width 0.1524) (layer F.Cu) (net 12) (status 80000))
 (segment (start 124.714 85.344) (end 124.968 85.598) (width 0.1524) (layer F.Cu) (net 12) (status 80000))
 (segment (start 124.968 85.598) (end 124.968 85.852) (width 0.1524) (layer F.Cu) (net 12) (status 80000))
 (segment (start 124.968 85.852) (end 130.048 90.932) (width 0.1524) (layer F.Cu) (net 12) (status 80000))
 (segment (start 130.048 90.932) (end 130.048 96.52) (width 0.1524) (layer F.Cu) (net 12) (status 80000))
 (via (at 130.048 96.52) (size 0.6858) (layers F.Cu B.Cu) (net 12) (status 80000))
 (segment (start 130.048 96.52) (end 133.604 100.076) (width 0.1524) (layer B.Cu) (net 12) (status 80000))
 (segment (start 117.856 77.724) (end 119.888 79.756) (width 0.1524) (layer F.Cu) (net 13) (status 80000))
 (segment (start 119.888 79.756) (end 119.888 81.534) (width 0.1524) (layer F.Cu) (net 13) (status 80000))
 (segment (start 119.888 81.534) (end 122.174 83.82) (width 0.1524) (layer F.Cu) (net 13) (status 80000))
 (segment (start 122.174 83.82) (end 122.174 85.344) (width 0.1524) (layer F.Cu) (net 13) (status 80000))
 (segment (start 122.174 85.344) (end 122.428 85.598) (width 0.1524) (layer F.Cu) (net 13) (status 80000))
 (segment (start 122.428 85.598) (end 122.428 85.852) (width 0.1524) (layer F.Cu) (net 13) (status 80000))
 (segment (start 122.428 85.852) (end 129.032 92.456) (width 0.1524) (layer F.Cu) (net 13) (status 80000))
 (segment (start 129.032 92.456) (end 129.032 92.964) (width 0.1524) (layer F.Cu) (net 13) (status 80000))
 (via (at 129.032 92.964) (size 0.6858) (layers F.Cu B.Cu) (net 13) (status 80000))
 (segment (start 129.032 92.964) (end 136.144 100.076) (width 0.1524) (layer B.Cu) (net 13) (status 80000))
 (segment (start 112.776 77.724) (end 114.046 78.994) (width 0.1524) (layer F.Cu) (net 14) (status 80000))
 (segment (start 114.046 78.994) (end 114.554 78.994) (width 0.1524) (layer F.Cu) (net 14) (status 80000))
 (segment (start 114.554 78.994) (end 119.634 84.074) (width 0.1524) (layer F.Cu) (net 14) (status 80000))
 (segment (start 119.634 84.074) (end 119.634 85.344) (width 0.1524) (layer F.Cu) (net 14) (status 80000))
 (segment (start 119.634 85.344) (end 119.888 85.598) (width 0.1524) (layer F.Cu) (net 14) (status 80000))
 (segment (start 119.888 85.598) (end 119.888 85.852) (width 0.1524) (layer F.Cu) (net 14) (status 80000))
 (segment (start 119.888 85.852) (end 120.65 86.614) (width 0.1524) (layer F.Cu) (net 14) (status 80000))
 (via (at 120.65 86.614) (size 0.6858) (layers F.Cu B.Cu) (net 14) (status 80000))
 (segment (start 120.65 86.614) (end 126.238 92.202) (width 0.1524) (layer B.Cu) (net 14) (status 80000))
 (segment (start 126.238 92.202) (end 129.54 92.202) (width 0.1524) (layer B.Cu) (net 14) (status 80000))
 (segment (start 129.54 92.202) (end 136.144 98.806) (width 0.1524) (layer B.Cu) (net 14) (status 80000))
 (segment (start 136.144 98.806) (end 136.652 98.806) (width 0.1524) (layer B.Cu) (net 14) (status 80000))
 (segment (start 136.652 98.806) (end 136.906 99.06) (width 0.1524) (layer B.Cu) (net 14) (status 80000))
 (segment (start 136.906 99.06) (end 137.16 99.06) (width 0.1524) (layer B.Cu) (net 14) (status 80000))
 (segment (start 137.16 99.06) (end 138.176 100.076) (width 0.1524) (layer B.Cu) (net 14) (status 80000))
 (segment (start 138.176 100.076) (end 138.684 100.076) (width 0.1524) (layer B.Cu) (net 14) (status 80000))
 (segment (start 125.476 77.724) (end 119.634 83.566) (width 0.1524) (layer B.Cu) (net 22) (status 80000))
 (segment (start 119.634 83.566) (end 112.776 83.566) (width 0.1524) (layer B.Cu) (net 22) (status 80000))
 (segment (start 112.776 83.566) (end 112.522 83.82) (width 0.1524) (layer B.Cu) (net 22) (status 80000))
 (segment (start 112.522 83.82) (end 112.268 83.82) (width 0.1524) (layer B.Cu) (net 22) (status 80000))
 (segment (start 112.268 83.82) (end 111.252 84.836) (width 0.1524) (layer B.Cu) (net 22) (status 80000))
 (segment (start 111.252 84.836) (end 110.744 84.836) (width 0.1524) (layer B.Cu) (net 22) (status 80000))
 (segment (start 115.316 77.724) (end 118.618 81.026) (width 0.1524) (layer B.Cu) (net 20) (status 80000))
 (segment (start 118.618 81.026) (end 120.65 81.026) (width 0.1524) (layer B.Cu) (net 20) (status 80000))
 (via (at 120.65 81.026) (size 0.6858) (layers F.Cu B.Cu) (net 20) (status 80000))
 (segment (start 120.65 81.026) (end 122.174 82.55) (width 0.1524) (layer F.Cu) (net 20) (status 80000))
 (via (at 122.174 82.55) (size 0.6858) (layers F.Cu B.Cu) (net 20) (status 80000))
 (segment (start 122.174 82.55) (end 123.19 83.566) (width 0.1524) (layer B.Cu) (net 20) (status 80000))
 (segment (start 123.19 83.566) (end 136.652 83.566) (width 0.1524) (layer B.Cu) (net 20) (status 80000))
 (segment (start 136.652 83.566) (end 136.906 83.82) (width 0.1524) (layer B.Cu) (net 20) (status 80000))
 (segment (start 136.906 83.82) (end 137.16 83.82) (width 0.1524) (layer B.Cu) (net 20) (status 80000))
 (segment (start 137.16 83.82) (end 138.176 84.836) (width 0.1524) (layer B.Cu) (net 20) (status 80000))
 (segment (start 138.176 84.836) (end 138.684 84.836) (width 0.1524) (layer B.Cu) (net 20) (status 80000))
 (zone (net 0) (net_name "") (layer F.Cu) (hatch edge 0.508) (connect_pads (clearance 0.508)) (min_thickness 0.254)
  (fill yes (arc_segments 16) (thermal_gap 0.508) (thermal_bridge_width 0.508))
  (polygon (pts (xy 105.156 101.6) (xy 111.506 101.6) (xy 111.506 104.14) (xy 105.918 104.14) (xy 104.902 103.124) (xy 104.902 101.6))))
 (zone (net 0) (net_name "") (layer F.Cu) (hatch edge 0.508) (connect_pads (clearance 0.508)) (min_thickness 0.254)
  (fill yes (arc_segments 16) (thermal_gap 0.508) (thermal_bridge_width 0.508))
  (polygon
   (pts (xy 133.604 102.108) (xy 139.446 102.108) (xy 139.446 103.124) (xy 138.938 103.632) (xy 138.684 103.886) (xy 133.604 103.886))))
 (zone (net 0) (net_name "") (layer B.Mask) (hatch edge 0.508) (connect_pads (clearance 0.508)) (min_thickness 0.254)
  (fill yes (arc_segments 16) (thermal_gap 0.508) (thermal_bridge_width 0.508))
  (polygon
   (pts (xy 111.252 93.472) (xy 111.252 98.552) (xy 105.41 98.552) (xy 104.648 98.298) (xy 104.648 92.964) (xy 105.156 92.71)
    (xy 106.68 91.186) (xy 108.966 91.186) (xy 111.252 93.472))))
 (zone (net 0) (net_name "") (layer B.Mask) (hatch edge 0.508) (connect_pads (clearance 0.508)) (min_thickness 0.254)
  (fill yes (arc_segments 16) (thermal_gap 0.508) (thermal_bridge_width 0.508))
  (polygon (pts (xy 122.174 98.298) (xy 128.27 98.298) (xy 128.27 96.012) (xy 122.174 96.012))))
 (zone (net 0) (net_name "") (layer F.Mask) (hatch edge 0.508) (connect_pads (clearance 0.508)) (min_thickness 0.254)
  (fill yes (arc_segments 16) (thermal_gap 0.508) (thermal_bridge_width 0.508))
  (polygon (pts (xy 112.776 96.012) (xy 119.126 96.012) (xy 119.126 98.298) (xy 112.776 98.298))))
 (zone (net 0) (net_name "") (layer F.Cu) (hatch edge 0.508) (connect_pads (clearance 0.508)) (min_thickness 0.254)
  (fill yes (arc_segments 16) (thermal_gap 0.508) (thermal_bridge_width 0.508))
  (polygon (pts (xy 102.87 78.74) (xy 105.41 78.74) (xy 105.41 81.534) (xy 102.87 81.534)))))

